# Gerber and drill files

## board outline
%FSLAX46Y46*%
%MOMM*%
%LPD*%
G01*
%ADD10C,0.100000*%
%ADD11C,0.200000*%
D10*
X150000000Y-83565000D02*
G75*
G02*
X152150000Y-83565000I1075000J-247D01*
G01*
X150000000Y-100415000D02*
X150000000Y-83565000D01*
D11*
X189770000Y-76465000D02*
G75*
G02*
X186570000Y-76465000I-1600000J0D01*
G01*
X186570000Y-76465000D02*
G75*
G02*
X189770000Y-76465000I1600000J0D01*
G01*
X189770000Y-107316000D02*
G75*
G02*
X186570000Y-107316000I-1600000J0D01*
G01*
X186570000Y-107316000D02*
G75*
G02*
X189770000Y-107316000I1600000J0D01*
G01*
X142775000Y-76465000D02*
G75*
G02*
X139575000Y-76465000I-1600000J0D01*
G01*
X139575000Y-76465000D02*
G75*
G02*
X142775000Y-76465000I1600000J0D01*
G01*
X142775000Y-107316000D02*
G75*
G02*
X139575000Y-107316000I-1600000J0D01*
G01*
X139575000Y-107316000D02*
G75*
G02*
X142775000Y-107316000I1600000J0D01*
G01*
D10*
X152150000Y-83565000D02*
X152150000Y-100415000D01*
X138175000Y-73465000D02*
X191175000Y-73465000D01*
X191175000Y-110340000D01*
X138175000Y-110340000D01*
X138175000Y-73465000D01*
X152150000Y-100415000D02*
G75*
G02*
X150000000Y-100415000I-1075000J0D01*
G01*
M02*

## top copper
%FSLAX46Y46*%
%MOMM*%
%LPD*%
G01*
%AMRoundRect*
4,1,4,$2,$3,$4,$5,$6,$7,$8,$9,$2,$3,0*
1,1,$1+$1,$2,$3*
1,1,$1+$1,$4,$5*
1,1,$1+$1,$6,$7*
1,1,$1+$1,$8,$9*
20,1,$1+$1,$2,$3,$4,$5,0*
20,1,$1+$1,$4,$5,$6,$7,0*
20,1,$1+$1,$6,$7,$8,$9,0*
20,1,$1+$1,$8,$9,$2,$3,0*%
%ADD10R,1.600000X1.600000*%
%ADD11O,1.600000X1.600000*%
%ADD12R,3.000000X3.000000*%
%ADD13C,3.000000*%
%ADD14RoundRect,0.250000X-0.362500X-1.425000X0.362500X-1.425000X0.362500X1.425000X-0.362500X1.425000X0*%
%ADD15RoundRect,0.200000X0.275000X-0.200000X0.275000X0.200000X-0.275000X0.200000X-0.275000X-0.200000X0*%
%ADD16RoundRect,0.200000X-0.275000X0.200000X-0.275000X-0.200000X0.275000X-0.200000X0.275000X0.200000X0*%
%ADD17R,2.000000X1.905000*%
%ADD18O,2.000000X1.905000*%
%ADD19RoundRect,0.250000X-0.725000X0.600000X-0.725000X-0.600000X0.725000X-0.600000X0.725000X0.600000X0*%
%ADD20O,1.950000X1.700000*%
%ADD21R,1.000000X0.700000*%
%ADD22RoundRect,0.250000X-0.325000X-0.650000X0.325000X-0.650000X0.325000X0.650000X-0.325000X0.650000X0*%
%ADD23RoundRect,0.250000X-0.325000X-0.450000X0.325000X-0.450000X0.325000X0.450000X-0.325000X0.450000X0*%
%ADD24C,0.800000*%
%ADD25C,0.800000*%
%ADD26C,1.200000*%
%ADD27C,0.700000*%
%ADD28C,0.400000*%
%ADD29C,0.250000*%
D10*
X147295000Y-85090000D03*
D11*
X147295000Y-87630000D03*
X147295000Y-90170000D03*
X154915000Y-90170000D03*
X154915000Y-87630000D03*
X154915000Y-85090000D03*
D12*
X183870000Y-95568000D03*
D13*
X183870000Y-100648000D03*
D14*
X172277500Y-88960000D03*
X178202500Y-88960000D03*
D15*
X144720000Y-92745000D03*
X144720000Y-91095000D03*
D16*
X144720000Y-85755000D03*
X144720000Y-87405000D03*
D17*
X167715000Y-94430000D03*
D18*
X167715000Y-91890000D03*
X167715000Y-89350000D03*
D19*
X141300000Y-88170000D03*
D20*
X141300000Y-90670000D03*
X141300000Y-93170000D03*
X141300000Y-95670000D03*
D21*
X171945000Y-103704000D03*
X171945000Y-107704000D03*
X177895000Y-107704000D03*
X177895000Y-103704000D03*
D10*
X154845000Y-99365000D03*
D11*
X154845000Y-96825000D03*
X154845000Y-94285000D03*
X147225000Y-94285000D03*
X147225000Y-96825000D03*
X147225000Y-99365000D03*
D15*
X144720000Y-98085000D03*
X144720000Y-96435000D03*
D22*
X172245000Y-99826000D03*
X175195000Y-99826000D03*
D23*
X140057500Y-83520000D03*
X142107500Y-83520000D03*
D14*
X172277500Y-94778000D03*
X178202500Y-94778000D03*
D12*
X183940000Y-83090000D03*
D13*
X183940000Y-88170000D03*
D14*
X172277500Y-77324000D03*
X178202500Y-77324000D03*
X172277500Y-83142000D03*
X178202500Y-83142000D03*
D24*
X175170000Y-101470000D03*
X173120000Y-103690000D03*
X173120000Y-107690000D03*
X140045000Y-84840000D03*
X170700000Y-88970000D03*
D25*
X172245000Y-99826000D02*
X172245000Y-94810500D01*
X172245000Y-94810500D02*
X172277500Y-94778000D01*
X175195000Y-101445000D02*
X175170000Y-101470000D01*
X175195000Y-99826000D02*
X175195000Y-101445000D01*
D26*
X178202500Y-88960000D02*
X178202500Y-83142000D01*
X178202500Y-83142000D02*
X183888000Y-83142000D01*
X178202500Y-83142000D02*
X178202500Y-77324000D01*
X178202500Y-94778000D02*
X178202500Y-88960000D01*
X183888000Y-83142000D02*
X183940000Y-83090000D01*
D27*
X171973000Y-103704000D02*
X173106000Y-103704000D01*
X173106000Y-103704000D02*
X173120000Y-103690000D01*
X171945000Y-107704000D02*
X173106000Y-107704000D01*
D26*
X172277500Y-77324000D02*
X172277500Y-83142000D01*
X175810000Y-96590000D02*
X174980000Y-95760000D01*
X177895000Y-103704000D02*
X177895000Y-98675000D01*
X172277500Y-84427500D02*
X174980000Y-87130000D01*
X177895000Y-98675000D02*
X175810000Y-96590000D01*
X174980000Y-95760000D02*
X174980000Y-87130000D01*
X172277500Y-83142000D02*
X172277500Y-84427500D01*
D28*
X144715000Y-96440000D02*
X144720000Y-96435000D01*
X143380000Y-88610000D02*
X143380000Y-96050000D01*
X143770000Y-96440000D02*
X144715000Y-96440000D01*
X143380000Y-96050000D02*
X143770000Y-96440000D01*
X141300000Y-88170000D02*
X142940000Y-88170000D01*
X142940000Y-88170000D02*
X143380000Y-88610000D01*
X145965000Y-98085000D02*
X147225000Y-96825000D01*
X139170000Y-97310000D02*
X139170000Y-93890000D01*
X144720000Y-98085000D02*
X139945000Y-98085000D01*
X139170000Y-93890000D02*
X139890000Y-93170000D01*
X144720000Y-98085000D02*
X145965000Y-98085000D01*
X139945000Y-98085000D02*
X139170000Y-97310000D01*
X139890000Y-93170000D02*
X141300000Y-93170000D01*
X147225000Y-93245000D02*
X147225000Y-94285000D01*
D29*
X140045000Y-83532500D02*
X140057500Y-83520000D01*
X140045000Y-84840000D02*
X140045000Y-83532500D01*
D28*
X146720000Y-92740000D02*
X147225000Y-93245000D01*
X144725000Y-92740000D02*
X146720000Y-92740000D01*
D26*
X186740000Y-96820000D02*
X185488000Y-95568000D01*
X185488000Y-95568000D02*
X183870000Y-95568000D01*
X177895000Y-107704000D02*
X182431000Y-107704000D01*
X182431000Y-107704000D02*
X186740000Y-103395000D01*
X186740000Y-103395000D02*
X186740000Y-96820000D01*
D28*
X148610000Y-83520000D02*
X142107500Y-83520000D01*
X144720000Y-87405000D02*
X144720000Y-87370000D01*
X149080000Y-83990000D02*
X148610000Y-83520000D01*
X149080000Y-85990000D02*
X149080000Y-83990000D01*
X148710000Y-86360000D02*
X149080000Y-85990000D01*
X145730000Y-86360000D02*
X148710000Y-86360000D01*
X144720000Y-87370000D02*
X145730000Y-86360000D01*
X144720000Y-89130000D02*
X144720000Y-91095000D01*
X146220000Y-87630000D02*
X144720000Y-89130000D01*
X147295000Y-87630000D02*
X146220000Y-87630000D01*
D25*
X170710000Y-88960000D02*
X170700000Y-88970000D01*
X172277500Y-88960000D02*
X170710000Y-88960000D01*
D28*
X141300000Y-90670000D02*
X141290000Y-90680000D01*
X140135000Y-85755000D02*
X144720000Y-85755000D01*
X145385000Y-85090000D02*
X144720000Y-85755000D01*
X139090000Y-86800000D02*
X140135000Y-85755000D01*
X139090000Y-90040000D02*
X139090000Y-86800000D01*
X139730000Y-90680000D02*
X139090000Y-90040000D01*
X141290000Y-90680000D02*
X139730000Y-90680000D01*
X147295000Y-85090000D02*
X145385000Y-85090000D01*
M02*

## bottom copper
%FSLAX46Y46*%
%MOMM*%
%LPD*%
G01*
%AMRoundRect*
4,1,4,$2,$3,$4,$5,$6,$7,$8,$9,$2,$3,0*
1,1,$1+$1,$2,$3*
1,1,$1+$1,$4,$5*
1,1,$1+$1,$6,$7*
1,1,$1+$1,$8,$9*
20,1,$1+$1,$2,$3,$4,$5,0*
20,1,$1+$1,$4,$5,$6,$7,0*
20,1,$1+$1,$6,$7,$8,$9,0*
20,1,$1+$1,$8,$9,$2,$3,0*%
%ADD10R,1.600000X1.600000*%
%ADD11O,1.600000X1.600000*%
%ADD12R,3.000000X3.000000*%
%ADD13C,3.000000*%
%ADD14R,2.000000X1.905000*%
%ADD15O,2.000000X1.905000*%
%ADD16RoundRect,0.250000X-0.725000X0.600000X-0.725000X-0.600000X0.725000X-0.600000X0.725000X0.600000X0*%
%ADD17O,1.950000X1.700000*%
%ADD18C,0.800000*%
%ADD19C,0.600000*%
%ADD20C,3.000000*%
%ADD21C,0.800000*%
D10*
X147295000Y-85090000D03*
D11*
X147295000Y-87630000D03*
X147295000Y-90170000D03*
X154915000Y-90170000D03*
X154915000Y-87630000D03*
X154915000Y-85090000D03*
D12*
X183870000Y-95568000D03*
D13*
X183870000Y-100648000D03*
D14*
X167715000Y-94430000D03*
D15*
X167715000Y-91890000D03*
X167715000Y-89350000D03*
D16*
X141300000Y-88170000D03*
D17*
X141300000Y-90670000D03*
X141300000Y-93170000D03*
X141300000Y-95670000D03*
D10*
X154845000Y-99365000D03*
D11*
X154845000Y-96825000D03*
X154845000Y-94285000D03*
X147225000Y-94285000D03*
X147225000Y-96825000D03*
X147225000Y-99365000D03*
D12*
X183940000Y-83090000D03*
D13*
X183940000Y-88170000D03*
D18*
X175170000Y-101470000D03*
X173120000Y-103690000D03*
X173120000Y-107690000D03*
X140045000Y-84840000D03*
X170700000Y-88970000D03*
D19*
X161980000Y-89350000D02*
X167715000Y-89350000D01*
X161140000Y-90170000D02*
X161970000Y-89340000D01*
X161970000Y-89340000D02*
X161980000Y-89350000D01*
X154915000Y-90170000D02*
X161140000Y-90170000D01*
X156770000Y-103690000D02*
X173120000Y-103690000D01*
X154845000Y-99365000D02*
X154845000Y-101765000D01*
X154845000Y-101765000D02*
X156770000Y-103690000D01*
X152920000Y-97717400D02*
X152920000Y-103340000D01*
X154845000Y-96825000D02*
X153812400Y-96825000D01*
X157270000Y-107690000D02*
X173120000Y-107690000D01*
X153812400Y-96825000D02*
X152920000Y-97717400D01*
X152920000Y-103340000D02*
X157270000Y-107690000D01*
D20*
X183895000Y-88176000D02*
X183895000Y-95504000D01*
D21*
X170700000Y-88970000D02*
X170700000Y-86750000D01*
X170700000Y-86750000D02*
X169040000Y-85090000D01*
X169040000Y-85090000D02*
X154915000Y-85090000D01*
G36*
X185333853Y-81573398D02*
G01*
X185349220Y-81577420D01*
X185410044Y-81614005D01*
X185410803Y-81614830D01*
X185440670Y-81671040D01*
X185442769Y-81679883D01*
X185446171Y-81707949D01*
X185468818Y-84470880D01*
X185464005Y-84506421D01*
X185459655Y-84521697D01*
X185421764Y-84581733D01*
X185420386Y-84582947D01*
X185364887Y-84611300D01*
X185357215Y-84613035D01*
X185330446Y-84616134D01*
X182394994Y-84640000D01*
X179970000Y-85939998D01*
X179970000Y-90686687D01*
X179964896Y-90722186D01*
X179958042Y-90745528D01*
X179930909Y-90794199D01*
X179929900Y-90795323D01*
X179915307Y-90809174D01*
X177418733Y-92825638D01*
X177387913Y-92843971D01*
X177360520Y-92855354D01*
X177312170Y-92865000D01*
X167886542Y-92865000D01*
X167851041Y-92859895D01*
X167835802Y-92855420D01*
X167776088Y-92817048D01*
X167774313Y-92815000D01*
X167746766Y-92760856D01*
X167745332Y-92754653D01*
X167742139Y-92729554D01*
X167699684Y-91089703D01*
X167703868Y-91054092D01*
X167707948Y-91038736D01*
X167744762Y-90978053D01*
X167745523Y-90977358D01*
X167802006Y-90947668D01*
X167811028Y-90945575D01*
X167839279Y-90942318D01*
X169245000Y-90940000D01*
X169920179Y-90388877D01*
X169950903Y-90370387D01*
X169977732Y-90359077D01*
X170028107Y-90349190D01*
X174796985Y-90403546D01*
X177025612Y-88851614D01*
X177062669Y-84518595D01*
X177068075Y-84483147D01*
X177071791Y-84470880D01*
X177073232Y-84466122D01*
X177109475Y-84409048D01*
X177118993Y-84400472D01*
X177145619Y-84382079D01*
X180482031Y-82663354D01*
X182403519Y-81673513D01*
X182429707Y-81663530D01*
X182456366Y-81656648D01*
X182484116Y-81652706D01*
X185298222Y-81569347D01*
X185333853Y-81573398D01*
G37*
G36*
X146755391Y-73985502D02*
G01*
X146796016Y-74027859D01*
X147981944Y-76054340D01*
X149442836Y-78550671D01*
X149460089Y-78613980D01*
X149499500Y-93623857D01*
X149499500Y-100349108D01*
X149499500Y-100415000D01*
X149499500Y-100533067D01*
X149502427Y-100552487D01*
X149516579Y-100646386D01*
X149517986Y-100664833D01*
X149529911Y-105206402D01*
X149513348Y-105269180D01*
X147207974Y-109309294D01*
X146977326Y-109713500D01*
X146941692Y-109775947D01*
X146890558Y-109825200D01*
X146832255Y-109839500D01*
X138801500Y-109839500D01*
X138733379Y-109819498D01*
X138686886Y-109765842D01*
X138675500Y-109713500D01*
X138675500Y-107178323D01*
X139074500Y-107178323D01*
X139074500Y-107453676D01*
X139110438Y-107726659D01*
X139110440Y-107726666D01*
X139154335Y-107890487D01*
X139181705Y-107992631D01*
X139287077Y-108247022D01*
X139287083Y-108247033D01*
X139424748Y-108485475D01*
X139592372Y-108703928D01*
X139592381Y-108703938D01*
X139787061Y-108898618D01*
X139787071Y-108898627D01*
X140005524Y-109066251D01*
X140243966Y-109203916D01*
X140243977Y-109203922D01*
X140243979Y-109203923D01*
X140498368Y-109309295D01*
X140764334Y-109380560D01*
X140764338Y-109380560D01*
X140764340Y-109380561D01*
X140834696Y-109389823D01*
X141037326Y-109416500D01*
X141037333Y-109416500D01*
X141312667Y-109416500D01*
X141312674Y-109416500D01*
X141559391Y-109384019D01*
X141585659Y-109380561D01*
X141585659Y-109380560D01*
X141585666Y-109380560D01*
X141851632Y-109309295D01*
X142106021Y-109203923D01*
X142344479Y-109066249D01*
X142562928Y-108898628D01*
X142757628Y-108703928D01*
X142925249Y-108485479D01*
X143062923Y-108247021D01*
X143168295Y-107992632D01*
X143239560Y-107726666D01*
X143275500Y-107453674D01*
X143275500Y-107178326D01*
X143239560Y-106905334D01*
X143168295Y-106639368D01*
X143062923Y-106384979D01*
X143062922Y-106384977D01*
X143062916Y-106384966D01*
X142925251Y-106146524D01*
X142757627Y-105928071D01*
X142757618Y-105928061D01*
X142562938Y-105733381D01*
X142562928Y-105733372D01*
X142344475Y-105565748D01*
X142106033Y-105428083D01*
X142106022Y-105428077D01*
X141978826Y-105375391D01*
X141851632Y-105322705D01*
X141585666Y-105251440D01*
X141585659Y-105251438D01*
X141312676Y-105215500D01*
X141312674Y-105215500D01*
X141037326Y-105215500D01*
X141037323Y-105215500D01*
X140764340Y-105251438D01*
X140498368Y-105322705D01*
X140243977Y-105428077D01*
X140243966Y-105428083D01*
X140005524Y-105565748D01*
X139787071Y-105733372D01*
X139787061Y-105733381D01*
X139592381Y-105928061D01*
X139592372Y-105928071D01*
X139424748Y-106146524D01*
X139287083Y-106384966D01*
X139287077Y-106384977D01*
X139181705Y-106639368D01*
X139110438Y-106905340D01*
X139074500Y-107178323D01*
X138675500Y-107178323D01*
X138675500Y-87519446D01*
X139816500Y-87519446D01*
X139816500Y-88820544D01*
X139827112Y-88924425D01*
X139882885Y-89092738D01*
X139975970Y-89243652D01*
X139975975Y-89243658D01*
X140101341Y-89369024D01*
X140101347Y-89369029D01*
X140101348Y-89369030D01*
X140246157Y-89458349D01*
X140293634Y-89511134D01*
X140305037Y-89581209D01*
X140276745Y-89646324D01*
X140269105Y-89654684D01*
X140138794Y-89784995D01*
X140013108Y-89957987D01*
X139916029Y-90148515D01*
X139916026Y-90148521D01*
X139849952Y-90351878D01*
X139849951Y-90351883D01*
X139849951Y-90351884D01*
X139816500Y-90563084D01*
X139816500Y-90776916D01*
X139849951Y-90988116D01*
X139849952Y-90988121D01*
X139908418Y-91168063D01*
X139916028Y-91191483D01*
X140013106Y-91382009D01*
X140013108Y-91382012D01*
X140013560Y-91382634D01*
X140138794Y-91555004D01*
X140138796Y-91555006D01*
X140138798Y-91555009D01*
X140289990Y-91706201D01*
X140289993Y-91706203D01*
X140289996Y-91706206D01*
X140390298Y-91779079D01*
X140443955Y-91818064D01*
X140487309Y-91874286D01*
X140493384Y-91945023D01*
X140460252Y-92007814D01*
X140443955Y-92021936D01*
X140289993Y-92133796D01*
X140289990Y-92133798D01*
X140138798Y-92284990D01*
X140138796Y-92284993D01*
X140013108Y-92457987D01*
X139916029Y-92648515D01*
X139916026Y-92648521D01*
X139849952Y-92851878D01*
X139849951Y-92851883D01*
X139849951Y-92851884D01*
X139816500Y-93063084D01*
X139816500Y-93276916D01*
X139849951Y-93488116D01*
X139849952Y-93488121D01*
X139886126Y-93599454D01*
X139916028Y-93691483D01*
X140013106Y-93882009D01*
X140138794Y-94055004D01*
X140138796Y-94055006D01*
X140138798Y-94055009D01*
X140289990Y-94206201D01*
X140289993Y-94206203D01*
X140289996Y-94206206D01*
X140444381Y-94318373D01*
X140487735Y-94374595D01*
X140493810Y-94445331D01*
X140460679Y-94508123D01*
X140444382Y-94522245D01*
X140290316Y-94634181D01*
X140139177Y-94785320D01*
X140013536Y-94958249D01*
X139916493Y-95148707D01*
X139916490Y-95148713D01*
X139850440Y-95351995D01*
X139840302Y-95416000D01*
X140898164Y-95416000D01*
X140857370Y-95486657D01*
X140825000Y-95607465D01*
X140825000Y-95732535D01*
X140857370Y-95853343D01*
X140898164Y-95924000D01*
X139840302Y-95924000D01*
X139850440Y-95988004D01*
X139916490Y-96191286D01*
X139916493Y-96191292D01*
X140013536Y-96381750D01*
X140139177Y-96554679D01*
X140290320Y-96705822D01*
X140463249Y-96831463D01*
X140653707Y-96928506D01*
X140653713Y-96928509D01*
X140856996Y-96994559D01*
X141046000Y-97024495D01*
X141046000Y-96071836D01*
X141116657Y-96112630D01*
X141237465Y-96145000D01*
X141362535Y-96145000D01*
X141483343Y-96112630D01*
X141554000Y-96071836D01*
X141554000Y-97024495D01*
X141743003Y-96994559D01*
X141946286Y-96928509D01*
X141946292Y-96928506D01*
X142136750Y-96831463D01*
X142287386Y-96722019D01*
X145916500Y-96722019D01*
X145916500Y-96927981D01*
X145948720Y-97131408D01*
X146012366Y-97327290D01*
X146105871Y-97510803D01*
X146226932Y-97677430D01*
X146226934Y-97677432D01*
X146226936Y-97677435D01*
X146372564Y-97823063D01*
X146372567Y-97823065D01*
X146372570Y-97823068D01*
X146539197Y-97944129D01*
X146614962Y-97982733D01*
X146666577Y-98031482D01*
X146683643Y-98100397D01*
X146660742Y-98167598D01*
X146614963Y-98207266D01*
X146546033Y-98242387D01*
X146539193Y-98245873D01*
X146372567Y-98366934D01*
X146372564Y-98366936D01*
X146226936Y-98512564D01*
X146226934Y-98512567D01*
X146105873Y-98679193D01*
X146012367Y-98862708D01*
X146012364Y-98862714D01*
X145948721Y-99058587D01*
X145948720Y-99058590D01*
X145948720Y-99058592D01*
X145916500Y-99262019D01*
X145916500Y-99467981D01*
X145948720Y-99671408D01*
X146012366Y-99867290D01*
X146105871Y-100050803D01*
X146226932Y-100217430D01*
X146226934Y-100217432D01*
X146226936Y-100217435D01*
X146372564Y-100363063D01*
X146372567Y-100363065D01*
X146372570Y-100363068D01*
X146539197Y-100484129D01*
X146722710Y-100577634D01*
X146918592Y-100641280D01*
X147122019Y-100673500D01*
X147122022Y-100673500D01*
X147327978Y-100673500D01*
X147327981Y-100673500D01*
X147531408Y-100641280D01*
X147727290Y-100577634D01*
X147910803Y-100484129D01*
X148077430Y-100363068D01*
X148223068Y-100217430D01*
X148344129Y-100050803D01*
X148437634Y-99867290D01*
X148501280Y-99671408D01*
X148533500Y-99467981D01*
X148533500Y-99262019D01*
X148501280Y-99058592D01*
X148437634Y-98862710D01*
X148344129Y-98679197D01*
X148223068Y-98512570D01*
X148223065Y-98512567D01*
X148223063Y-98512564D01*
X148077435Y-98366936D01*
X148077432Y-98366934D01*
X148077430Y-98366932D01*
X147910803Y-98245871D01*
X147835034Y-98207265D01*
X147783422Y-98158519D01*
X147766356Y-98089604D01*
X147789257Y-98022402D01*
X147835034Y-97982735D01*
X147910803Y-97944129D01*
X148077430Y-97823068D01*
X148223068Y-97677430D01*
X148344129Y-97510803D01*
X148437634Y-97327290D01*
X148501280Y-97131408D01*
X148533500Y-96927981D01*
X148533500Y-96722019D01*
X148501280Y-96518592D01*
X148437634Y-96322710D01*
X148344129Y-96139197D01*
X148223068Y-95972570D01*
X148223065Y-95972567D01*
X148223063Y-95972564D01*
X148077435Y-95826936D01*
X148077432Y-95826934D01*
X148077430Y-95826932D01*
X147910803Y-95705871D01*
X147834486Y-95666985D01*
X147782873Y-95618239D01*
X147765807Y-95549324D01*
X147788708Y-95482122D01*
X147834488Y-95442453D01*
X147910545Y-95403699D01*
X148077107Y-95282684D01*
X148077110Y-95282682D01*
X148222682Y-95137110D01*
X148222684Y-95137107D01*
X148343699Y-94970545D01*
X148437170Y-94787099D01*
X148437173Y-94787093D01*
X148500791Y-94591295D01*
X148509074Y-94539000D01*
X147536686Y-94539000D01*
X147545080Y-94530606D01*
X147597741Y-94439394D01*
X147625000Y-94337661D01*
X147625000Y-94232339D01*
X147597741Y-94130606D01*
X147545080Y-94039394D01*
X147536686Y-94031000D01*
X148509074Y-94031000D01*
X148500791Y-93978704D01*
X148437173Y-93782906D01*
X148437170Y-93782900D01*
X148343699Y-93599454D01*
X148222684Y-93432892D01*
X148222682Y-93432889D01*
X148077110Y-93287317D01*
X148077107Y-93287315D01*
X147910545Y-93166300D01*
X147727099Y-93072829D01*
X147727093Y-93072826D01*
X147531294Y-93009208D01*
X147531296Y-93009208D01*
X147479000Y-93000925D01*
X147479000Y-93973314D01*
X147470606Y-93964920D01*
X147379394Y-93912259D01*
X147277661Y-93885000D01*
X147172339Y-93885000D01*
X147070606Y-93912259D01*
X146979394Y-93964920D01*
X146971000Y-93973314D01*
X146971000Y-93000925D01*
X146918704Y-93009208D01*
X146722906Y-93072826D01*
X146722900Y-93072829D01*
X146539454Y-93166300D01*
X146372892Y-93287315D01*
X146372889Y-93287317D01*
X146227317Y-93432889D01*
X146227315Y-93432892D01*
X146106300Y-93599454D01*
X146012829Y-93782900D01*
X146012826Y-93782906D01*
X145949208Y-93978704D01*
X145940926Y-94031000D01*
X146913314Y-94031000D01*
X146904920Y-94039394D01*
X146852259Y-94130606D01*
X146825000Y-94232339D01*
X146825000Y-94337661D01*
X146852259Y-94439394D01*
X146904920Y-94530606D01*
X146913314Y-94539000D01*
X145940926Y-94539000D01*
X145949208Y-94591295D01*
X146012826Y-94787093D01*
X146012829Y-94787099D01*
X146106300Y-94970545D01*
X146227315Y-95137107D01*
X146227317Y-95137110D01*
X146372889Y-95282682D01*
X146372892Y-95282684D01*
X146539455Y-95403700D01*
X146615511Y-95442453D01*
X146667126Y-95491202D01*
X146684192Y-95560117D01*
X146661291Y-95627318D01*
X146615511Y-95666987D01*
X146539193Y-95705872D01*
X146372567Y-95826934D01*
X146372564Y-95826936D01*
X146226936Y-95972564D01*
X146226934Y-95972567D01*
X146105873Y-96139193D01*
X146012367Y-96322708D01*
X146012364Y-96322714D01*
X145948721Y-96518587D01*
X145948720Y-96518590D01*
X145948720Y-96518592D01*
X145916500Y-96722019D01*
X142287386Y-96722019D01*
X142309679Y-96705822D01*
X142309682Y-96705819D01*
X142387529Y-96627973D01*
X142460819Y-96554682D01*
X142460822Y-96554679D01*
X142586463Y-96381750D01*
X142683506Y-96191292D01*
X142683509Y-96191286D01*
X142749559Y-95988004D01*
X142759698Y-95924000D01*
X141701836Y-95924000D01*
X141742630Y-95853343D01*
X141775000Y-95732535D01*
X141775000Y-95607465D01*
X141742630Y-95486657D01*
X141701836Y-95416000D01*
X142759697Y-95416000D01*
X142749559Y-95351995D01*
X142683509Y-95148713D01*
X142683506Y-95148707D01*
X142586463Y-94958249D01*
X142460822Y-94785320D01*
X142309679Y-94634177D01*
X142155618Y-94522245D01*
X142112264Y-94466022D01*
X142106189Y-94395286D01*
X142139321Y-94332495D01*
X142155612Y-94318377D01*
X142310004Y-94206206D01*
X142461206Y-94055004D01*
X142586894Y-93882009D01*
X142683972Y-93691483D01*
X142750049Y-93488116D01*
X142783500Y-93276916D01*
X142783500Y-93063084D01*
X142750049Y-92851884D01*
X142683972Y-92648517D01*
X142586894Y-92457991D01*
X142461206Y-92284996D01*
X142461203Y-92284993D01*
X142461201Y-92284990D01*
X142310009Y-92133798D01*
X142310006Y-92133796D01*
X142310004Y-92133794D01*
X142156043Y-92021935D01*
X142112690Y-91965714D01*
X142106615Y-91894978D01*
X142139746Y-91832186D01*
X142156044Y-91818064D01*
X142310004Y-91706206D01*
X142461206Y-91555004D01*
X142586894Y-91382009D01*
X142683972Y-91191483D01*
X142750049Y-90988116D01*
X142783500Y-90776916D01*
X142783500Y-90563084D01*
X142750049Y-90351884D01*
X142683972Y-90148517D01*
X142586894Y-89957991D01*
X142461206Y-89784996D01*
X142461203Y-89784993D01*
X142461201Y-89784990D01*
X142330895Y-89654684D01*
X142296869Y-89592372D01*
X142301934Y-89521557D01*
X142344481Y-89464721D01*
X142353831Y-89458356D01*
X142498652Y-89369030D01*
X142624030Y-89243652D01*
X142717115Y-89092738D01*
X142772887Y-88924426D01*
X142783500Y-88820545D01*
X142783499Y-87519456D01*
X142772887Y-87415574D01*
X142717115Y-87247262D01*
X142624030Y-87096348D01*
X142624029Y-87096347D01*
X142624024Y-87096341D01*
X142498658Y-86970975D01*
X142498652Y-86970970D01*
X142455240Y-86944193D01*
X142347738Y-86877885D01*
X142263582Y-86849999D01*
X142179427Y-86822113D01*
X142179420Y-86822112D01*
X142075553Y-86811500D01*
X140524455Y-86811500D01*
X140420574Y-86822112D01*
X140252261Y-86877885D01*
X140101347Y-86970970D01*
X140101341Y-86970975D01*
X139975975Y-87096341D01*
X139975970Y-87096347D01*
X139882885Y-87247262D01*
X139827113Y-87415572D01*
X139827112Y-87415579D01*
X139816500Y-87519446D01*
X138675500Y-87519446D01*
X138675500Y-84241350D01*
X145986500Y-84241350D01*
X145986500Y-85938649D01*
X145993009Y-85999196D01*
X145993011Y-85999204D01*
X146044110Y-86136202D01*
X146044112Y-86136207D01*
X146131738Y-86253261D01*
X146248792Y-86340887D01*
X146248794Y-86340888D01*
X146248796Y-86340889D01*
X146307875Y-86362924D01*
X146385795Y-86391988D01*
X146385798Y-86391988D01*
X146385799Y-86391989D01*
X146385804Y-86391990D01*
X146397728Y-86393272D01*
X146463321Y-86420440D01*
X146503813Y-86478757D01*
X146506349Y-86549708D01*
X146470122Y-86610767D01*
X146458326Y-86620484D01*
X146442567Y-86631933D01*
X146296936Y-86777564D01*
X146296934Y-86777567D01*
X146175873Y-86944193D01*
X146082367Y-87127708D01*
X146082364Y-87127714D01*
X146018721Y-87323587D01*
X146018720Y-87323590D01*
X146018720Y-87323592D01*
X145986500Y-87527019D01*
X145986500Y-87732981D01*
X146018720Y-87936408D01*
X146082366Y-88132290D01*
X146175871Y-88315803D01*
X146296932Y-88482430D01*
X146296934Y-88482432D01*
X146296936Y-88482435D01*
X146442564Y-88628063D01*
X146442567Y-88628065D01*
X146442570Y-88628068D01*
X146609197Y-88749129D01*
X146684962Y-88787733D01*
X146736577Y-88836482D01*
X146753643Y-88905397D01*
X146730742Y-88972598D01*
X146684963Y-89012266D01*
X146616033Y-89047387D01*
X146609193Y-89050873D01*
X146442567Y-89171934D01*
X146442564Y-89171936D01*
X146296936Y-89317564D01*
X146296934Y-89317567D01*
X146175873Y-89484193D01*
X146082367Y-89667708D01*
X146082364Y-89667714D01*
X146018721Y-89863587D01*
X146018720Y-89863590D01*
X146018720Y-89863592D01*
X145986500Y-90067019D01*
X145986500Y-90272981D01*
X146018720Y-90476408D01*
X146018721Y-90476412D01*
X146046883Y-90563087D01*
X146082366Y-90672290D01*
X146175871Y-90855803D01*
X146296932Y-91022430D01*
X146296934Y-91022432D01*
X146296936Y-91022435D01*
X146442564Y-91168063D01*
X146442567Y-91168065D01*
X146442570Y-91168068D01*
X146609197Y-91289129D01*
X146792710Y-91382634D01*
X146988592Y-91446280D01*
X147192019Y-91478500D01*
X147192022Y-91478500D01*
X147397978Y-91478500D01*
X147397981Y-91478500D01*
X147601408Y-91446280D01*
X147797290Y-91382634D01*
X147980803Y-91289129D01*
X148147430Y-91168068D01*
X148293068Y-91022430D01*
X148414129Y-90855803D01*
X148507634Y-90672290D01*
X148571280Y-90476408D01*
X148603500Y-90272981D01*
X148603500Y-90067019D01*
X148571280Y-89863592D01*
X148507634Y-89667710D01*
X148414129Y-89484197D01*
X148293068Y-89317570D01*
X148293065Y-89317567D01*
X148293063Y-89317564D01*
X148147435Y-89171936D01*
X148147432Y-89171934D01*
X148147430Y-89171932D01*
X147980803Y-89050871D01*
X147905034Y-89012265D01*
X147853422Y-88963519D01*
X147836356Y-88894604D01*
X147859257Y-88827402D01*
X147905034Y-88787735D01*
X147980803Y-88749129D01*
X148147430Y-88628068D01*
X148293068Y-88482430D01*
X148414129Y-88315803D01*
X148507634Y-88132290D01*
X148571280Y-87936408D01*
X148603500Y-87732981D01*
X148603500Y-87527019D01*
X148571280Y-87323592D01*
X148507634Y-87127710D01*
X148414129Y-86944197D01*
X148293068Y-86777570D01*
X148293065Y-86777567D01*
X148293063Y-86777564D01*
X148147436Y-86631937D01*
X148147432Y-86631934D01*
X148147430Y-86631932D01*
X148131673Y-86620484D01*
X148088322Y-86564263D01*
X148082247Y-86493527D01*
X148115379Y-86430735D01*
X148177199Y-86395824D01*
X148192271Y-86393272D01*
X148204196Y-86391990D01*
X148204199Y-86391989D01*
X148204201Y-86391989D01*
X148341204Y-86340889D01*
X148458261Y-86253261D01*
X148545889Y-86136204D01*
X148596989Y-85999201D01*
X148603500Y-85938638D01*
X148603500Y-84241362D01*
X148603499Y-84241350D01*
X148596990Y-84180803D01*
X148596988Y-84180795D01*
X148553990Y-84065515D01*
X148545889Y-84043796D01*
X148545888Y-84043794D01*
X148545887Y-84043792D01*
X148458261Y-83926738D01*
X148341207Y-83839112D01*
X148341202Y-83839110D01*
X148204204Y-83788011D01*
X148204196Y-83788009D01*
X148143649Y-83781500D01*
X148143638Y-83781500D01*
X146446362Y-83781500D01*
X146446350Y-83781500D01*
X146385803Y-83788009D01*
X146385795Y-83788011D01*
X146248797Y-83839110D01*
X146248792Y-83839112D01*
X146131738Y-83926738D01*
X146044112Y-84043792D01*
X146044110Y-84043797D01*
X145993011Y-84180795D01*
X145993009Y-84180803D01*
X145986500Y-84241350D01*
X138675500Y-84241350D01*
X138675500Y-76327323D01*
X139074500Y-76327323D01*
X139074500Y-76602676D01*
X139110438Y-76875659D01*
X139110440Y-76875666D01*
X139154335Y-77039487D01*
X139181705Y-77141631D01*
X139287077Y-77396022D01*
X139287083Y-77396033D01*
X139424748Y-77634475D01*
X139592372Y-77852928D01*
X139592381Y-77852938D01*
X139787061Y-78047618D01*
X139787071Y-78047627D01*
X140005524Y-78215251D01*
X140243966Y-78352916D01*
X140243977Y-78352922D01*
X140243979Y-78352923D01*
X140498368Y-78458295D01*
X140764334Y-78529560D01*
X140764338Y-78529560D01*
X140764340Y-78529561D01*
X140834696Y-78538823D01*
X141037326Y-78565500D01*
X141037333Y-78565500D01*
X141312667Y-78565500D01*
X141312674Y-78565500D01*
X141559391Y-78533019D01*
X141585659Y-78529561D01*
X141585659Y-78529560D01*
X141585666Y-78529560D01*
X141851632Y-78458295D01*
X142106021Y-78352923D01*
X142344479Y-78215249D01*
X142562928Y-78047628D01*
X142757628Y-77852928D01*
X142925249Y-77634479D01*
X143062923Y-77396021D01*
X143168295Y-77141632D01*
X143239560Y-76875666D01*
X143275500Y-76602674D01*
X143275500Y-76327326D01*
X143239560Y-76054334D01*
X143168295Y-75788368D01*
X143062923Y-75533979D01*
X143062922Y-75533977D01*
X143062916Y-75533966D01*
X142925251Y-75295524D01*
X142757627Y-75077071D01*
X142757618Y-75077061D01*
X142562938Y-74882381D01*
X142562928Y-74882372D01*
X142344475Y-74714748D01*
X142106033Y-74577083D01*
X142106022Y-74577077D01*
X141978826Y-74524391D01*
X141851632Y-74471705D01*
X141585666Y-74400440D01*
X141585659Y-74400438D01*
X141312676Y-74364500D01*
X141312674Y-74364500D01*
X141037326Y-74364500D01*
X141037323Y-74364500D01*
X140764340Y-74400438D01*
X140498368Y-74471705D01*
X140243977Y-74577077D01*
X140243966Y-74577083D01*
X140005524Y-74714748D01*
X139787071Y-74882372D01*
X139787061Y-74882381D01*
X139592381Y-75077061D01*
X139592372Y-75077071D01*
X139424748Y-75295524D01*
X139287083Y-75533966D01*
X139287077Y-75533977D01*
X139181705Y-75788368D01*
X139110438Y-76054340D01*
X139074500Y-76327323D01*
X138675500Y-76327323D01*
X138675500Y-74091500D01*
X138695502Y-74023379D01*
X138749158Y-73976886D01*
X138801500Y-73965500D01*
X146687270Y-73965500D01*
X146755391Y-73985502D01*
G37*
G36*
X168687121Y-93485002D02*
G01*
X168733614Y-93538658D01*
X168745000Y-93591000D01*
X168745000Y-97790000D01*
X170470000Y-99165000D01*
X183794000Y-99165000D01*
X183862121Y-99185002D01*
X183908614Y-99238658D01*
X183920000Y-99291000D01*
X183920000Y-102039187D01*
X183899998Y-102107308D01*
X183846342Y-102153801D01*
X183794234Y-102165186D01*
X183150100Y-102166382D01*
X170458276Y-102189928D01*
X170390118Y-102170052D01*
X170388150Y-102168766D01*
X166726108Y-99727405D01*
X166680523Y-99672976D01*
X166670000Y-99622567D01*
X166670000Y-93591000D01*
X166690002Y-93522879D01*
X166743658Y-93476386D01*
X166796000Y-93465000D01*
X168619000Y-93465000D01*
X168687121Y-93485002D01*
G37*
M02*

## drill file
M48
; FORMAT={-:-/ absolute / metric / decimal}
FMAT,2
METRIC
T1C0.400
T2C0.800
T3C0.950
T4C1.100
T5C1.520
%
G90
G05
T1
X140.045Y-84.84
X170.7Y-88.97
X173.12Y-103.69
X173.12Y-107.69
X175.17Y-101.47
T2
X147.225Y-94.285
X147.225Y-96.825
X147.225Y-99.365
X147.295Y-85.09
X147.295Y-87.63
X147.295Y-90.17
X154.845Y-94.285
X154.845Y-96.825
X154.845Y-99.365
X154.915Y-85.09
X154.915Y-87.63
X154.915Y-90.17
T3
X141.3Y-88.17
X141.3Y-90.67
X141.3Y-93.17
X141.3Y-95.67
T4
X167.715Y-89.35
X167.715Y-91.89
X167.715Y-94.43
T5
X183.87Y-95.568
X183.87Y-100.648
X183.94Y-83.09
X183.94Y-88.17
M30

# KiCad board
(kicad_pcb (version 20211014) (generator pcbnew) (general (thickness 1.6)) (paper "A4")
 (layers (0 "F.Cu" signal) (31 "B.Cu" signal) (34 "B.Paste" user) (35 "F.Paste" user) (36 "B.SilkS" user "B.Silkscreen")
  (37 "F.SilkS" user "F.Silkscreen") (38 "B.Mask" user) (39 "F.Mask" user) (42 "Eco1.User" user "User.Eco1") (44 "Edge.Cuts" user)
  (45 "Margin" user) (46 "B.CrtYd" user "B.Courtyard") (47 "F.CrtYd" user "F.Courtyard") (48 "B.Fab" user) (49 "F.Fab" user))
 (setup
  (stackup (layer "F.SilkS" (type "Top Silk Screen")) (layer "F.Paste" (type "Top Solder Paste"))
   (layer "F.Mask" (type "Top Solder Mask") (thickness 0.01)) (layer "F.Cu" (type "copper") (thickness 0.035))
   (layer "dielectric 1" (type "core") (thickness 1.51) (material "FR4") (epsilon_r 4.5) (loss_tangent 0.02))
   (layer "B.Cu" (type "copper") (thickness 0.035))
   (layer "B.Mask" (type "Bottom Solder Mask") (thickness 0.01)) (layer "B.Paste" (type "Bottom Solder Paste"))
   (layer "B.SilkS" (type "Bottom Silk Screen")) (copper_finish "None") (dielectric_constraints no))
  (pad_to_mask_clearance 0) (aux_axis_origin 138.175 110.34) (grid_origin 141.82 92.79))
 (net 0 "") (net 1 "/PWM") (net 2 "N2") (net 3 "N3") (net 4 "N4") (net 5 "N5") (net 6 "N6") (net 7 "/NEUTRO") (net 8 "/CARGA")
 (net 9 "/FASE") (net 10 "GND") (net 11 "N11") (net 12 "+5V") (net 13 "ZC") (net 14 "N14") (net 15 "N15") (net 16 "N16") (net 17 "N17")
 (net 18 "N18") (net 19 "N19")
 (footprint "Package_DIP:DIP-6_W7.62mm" (layer "F.Cu") (at 147.295 85.09)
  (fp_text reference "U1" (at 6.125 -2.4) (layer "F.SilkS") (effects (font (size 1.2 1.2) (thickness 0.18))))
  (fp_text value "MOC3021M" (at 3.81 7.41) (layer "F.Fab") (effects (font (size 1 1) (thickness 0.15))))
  (pad "1" thru_hole rect (at 0 0) (size 1.6 1.6) (drill 0.8) (layers *.Cu *.Mask) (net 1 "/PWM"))
  (pad "2" thru_hole oval (at 0 2.54) (size 1.6 1.6) (drill 0.8) (layers *.Cu *.Mask) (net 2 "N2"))
  (pad "3" thru_hole oval (at 0 5.08) (size 1.6 1.6) (drill 0.8) (layers *.Cu *.Mask) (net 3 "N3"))
  (pad "4" thru_hole oval (at 7.62 5.08) (size 1.6 1.6) (drill 0.8) (layers *.Cu *.Mask) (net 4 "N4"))
  (pad "5" thru_hole oval (at 7.62 2.54) (size 1.6 1.6) (drill 0.8) (layers *.Cu *.Mask) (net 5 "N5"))
  (pad "6" thru_hole oval (at 7.62 0) (size 1.6 1.6) (drill 0.8) (layers *.Cu *.Mask) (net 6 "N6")))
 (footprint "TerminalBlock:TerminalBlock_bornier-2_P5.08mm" (layer "F.Cu") (at 183.87 95.568 -90)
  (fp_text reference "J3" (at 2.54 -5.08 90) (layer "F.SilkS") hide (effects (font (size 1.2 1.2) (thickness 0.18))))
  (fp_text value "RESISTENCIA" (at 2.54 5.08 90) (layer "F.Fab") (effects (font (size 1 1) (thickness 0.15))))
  (pad "1" thru_hole rect (at 0 0 270) (size 3 3) (drill 1.52) (layers *.Cu *.Mask) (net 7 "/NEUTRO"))
  (pad "2" thru_hole circle (at 5.08 0 270) (size 3 3) (drill 1.52) (layers *.Cu *.Mask) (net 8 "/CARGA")))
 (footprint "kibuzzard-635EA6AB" (layer "F.Cu") (at 141.02 81.09)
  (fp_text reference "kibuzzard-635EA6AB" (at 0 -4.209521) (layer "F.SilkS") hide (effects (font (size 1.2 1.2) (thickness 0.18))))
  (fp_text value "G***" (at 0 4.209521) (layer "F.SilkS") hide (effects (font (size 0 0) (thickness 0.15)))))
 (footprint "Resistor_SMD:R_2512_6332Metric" (layer "F.Cu") (at 175.24 88.96)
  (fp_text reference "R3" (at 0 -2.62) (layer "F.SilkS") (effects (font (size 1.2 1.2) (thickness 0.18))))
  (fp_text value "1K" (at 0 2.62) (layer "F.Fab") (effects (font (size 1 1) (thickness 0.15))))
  (pad "1" smd roundrect (at -2.9625 0) (size 1.225 3.35) (layers "F.Cu" "F.Paste" "F.Mask") (roundrect_rratio 0.204082) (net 6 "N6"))
  (pad "2" smd roundrect (at 2.9625 0) (size 1.225 3.35) (layers "F.Cu" "F.Paste" "F.Mask") (roundrect_rratio 0.204082) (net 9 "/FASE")))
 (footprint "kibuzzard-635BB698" (layer "F.Cu") (at 189.41619 85.8 90)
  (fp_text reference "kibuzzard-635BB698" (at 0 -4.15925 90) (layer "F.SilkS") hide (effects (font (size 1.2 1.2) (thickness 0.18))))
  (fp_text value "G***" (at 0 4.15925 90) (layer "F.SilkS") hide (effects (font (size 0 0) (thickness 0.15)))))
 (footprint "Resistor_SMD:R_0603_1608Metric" (layer "F.Cu") (at 144.72 91.92 90)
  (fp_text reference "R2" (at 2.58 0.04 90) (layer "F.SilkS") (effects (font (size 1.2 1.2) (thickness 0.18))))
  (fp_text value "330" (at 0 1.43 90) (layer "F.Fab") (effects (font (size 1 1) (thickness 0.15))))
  (pad "1" smd roundrect (at -0.825 0 90) (size 0.8 0.95) (layers "F.Cu" "F.Paste" "F.Mask") (roundrect_rratio 0.25) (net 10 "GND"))
  (pad "2" smd roundrect (at 0.825 0 90) (size 0.8 0.95) (layers "F.Cu" "F.Paste" "F.Mask") (roundrect_rratio 0.25) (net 2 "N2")))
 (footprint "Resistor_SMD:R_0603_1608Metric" (layer "F.Cu") (at 144.72 86.58 -90)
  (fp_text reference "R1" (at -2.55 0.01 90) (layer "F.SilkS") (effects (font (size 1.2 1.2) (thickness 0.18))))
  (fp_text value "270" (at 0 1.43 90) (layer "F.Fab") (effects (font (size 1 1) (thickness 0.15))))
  (pad "1" smd roundrect (at -0.825 0 270) (size 0.8 0.95) (layers "F.Cu" "F.Paste" "F.Mask") (roundrect_rratio 0.25) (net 1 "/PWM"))
  (pad "2" smd roundrect (at 0.825 0 270) (size 0.8 0.95) (layers "F.Cu" "F.Paste" "F.Mask") (roundrect_rratio 0.25) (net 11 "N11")))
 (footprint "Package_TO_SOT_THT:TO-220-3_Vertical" (layer "F.Cu") (at 167.715 94.43 90)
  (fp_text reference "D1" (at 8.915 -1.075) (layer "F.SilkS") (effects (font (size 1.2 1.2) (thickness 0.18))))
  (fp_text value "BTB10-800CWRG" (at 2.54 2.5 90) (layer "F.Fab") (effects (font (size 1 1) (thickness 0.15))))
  (pad "1" thru_hole rect (at 0 0 90) (size 1.905 2) (drill 1.1) (layers *.Cu *.Mask) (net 8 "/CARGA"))
  (pad "2" thru_hole oval (at 2.54 0 90) (size 1.905 2) (drill 1.1) (layers *.Cu *.Mask) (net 9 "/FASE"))
  (pad "3" thru_hole oval (at 5.08 0 90) (size 1.905 2) (drill 1.1) (layers *.Cu *.Mask) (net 4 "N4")))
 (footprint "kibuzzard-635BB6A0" (layer "F.Cu") (at 189.42 98.01 90)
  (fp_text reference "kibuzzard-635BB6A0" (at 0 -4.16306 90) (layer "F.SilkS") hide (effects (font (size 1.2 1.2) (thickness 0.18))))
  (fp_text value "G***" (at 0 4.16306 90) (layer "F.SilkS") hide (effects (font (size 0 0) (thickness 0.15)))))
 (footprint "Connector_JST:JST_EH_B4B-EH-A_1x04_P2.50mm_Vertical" (layer "F.Cu") (at 141.3 88.17 -90)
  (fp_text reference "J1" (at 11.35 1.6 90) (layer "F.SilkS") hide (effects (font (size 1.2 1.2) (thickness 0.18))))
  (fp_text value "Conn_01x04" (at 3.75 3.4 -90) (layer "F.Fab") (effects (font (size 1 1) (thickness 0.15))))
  (pad "1" thru_hole roundrect (at 0 0 270) (size 1.7 1.95) (drill 0.95) (layers *.Cu *.Mask) (roundrect_rratio 0.147059) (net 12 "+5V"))
  (pad "2" thru_hole oval (at 2.5 0 270) (size 1.7 1.95) (drill 0.95) (layers *.Cu *.Mask) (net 1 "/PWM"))
  (pad "3" thru_hole oval (at 5 0 270) (size 1.7 1.95) (drill 0.95) (layers *.Cu *.Mask) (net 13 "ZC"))
  (pad "4" thru_hole oval (at 7.5 0 270) (size 1.7 1.95) (drill 0.95) (layers *.Cu *.Mask) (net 10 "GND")))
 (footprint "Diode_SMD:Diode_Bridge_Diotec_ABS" (layer "F.Cu") (at 174.92 105.704)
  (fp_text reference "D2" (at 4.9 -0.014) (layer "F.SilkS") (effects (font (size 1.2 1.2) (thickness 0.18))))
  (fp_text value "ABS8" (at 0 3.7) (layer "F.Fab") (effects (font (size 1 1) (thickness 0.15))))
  (pad "1" smd rect (at -2.975 -2) (size 1 0.7) (layers "F.Cu" "F.Paste" "F.Mask") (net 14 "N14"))
  (pad "2" smd rect (at -2.975 2) (size 1 0.7) (layers "F.Cu" "F.Paste" "F.Mask") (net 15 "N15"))
  (pad "3" smd rect (at 2.975 2) (size 1 0.7) (layers "F.Cu" "F.Paste" "F.Mask") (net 7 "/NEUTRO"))
  (pad "4" smd rect (at 2.975 -2) (size 1 0.7) (layers "F.Cu" "F.Paste" "F.Mask") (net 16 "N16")))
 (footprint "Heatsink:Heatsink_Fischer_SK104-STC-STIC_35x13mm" (layer "F.Cu") (at 163.48 91.96 90)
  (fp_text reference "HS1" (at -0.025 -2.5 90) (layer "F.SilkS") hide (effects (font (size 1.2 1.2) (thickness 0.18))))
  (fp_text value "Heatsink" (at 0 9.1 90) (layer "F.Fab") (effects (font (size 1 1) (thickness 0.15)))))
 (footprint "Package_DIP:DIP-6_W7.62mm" (layer "F.Cu") (at 154.845 99.365 180)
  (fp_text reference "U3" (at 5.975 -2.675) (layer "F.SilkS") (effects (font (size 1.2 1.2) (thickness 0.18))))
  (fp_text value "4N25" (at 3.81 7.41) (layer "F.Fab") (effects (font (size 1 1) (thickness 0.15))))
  (pad "1" thru_hole rect (at 0 0 180) (size 1.6 1.6) (drill 0.8) (layers *.Cu *.Mask) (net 14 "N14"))
  (pad "2" thru_hole oval (at 0 2.54 180) (size 1.6 1.6) (drill 0.8) (layers *.Cu *.Mask) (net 15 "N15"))
  (pad "3" thru_hole oval (at 0 5.08 180) (size 1.6 1.6) (drill 0.8) (layers *.Cu *.Mask) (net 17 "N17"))
  (pad "4" thru_hole oval (at 7.62 5.08 180) (size 1.6 1.6) (drill 0.8) (layers *.Cu *.Mask) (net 10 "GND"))
  (pad "5" thru_hole oval (at 7.62 2.54 180) (size 1.6 1.6) (drill 0.8) (layers *.Cu *.Mask) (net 13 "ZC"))
  (pad "6" thru_hole oval (at 7.62 0 180) (size 1.6 1.6) (drill 0.8) (layers *.Cu *.Mask) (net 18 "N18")))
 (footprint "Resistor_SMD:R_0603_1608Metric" (layer "F.Cu") (at 144.72 97.26 90)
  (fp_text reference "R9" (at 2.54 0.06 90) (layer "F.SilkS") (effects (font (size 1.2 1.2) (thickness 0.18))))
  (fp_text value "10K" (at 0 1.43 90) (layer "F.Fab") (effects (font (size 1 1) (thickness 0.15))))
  (pad "1" smd roundrect (at -0.825 0 90) (size 0.8 0.95) (layers "F.Cu" "F.Paste" "F.Mask") (roundrect_rratio 0.25) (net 13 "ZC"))
  (pad "2" smd roundrect (at 0.825 0 90) (size 0.8 0.95) (layers "F.Cu" "F.Paste" "F.Mask") (roundrect_rratio 0.25) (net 12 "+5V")))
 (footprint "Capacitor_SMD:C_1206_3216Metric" (layer "F.Cu") (at 173.72 99.826)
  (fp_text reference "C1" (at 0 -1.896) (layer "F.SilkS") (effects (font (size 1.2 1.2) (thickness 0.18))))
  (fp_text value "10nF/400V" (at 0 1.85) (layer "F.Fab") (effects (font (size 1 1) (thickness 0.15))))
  (pad "1" smd roundrect (at -1.475 0) (size 1.15 1.8) (layers "F.Cu" "F.Paste" "F.Mask") (roundrect_rratio 0.217391) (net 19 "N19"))
  (pad "2" smd roundrect (at 1.475 0) (size 1.15 1.8) (layers "F.Cu" "F.Paste" "F.Mask") (roundrect_rratio 0.217391) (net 8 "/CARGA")))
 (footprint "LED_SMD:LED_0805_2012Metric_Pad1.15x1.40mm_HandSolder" (layer "F.Cu") (at 141.0825 83.52)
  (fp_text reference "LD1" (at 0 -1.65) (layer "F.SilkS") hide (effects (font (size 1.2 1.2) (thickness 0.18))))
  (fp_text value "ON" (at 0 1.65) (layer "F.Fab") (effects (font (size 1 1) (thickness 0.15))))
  (pad "1" smd roundrect (at -1.025 0) (size 1.15 1.4) (layers "F.Cu" "F.Paste" "F.Mask") (roundrect_rratio 0.217391) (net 10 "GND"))
  (pad "2" smd roundrect (at 1.025 0) (size 1.15 1.4) (layers "F.Cu" "F.Paste" "F.Mask") (roundrect_rratio 0.217391) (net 11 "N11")))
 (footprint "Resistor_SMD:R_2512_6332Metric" (layer "F.Cu") (at 175.24 94.778)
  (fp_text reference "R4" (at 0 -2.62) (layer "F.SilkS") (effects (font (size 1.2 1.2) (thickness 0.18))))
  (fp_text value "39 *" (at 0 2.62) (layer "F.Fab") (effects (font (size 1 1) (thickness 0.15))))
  (pad "1" smd roundrect (at -2.9625 0) (size 1.225 3.35) (layers "F.Cu" "F.Paste" "F.Mask") (roundrect_rratio 0.204082) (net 19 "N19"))
  (pad "2" smd roundrect (at 2.9625 0) (size 1.225 3.35) (layers "F.Cu" "F.Paste" "F.Mask") (roundrect_rratio 0.204082) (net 9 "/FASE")))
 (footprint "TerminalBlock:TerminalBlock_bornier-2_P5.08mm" (layer "F.Cu") (at 183.94 83.09 -90)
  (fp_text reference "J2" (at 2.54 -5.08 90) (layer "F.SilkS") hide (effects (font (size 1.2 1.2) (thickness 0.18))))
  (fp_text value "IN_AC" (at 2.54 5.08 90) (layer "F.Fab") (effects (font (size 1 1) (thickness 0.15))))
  (pad "1" thru_hole rect (at 0 0 270) (size 3 3) (drill 1.52) (layers *.Cu *.Mask) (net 9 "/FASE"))
  (pad "2" thru_hole circle (at 5.08 0 270) (size 3 3) (drill 1.52) (layers *.Cu *.Mask) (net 7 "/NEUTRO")))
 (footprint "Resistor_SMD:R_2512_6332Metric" (layer "F.Cu") (at 175.24 77.324)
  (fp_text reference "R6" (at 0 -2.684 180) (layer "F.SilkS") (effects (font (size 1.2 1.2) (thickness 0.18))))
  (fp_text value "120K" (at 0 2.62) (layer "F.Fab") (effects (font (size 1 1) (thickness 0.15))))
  (pad "1" smd roundrect (at -2.9625 0) (size 1.225 3.35) (layers "F.Cu" "F.Paste" "F.Mask") (roundrect_rratio 0.204082) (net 16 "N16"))
  (pad "2" smd roundrect (at 2.9625 0) (size 1.225 3.35) (layers "F.Cu" "F.Paste" "F.Mask") (roundrect_rratio 0.204082) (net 9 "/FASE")))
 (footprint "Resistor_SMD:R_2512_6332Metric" (layer "F.Cu") (at 175.24 83.142)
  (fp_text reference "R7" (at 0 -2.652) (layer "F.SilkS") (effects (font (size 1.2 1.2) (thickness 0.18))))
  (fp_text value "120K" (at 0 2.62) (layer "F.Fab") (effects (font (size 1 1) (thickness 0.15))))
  (pad "1" smd roundrect (at -2.9625 0) (size 1.225 3.35) (layers "F.Cu" "F.Paste" "F.Mask") (roundrect_rratio 0.204082) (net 16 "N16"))
  (pad "2" smd roundrect (at 2.9625 0) (size 1.225 3.35) (layers "F.Cu" "F.Paste" "F.Mask") (roundrect_rratio 0.204082) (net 9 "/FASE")))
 (gr_arc (start 150 83.565) (mid 151.075 82.490247) (end 152.15 83.565) (layer "Edge.Cuts") (width 0.1))
 (gr_line (start 150 100.415) (end 150 83.565) (layer "Edge.Cuts") (width 0.1))
 (gr_circle (center 188.17 76.465) (end 189.77 76.465) (layer "Edge.Cuts") (width 0.2) (fill none))
 (gr_circle (center 188.17 107.316) (end 189.77 107.316) (layer "Edge.Cuts") (width 0.2) (fill none))
 (gr_circle (center 141.175 76.465) (end 142.775 76.465) (layer "Edge.Cuts") (width 0.2) (fill none))
 (gr_circle (center 141.175 107.316) (end 142.775 107.316) (layer "Edge.Cuts") (width 0.2) (fill none))
 (gr_line (start 152.15 83.565) (end 152.15 100.415) (layer "Edge.Cuts") (width 0.1))
 (gr_rect (start 138.175 73.465) (end 191.175 110.34) (layer "Edge.Cuts") (width 0.1) (fill none))
 (gr_arc (start 152.15 100.415) (mid 151.075 101.49) (end 150 100.415) (layer "Edge.Cuts") (width 0.1))
 (segment (start 172.245 99.826) (end 172.245 94.8105) (width 0.8) (layer "F.Cu") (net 19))
 (segment (start 172.245 94.8105) (end 172.2775 94.778) (width 0.8) (layer "F.Cu") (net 19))
 (segment (start 175.195 101.445) (end 175.17 101.47) (width 0.8) (layer "F.Cu") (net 8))
 (segment (start 175.195 99.826) (end 175.195 101.445) (width 0.8) (layer "F.Cu") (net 8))
 (via (at 175.17 101.47) (size 0.8) (drill 0.4) (layers "F.Cu" "B.Cu") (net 8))
 (segment (start 178.2025 88.96) (end 178.2025 83.142) (width 1.2) (layer "F.Cu") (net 9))
 (segment (start 178.2025 83.142) (end 183.888 83.142) (width 1.2) (layer "F.Cu") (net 9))
 (segment (start 178.2025 83.142) (end 178.2025 77.324) (width 1.2) (layer "F.Cu") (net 9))
 (segment (start 178.2025 94.778) (end 178.2025 88.96) (width 1.2) (layer "F.Cu") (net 9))
 (segment (start 183.888 83.142) (end 183.94 83.09) (width 1.2) (layer "F.Cu") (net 9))
 (segment (start 161.98 89.35) (end 167.715 89.35) (width 0.6) (layer "B.Cu") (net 4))
 (segment (start 161.14 90.17) (end 161.97 89.34) (width 0.6) (layer "B.Cu") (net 4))
 (segment (start 161.97 89.34) (end 161.98 89.35) (width 0.6) (layer "B.Cu") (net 4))
 (segment (start 154.915 90.17) (end 161.14 90.17) (width 0.6) (layer "B.Cu") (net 4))
 (segment (start 171.973 103.704) (end 173.106 103.704) (width 0.7) (layer "F.Cu") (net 14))
 (segment (start 173.106 103.704) (end 173.12 103.69) (width 0.7) (layer "F.Cu") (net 14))
 (via (at 173.12 103.69) (size 0.8) (drill 0.4) (layers "F.Cu" "B.Cu") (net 14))
 (segment (start 156.77 103.69) (end 173.12 103.69) (width 0.6) (layer "B.Cu") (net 14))
 (segment (start 154.845 99.365) (end 154.845 101.765) (width 0.6) (layer "B.Cu") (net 14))
 (segment (start 154.845 101.765) (end 156.77 103.69) (width 0.6) (layer "B.Cu") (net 14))
 (segment (start 171.945 107.704) (end 173.106 107.704) (width 0.7) (layer "F.Cu") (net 15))
 (via (at 173.12 107.69) (size 0.8) (drill 0.4) (layers "F.Cu" "B.Cu") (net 15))
 (segment (start 152.92 97.7174) (end 152.92 103.34) (width 0.6) (layer "B.Cu") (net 15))
 (segment (start 154.845 96.825) (end 153.8124 96.825) (width 0.6) (layer "B.Cu") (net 15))
 (segment (start 157.27 107.69) (end 173.12 107.69) (width 0.6) (layer "B.Cu") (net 15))
 (segment (start 153.8124 96.825) (end 152.92 97.7174) (width 0.6) (layer "B.Cu") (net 15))
 (segment (start 152.92 103.34) (end 157.27 107.69) (width 0.6) (layer "B.Cu") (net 15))
 (segment (start 172.2775 77.324) (end 172.2775 83.142) (width 1.2) (layer "F.Cu") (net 16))
 (segment (start 175.81 96.59) (end 174.98 95.76) (width 1.2) (layer "F.Cu") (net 16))
 (segment (start 177.895 103.704) (end 177.895 98.675) (width 1.2) (layer "F.Cu") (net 16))
 (segment (start 172.2775 84.4275) (end 174.98 87.13) (width 1.2) (layer "F.Cu") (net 16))
 (segment (start 177.895 98.675) (end 175.81 96.59) (width 1.2) (layer "F.Cu") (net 16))
 (segment (start 174.98 95.76) (end 174.98 87.13) (width 1.2) (layer "F.Cu") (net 16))
 (segment (start 172.2775 83.142) (end 172.2775 84.4275) (width 1.2) (layer "F.Cu") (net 16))
 (segment (start 144.715 96.44) (end 144.72 96.435) (width 0.4) (layer "F.Cu") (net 12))
 (segment (start 143.38 88.61) (end 143.38 96.05) (width 0.4) (layer "F.Cu") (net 12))
 (segment (start 143.77 96.44) (end 144.715 96.44) (width 0.4) (layer "F.Cu") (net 12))
 (segment (start 143.38 96.05) (end 143.77 96.44) (width 0.4) (layer "F.Cu") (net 12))
 (segment (start 141.3 88.17) (end 142.94 88.17) (width 0.4) (layer "F.Cu") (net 12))
 (segment (start 142.94 88.17) (end 143.38 88.61) (width 0.4) (layer "F.Cu") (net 12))
 (segment (start 145.965 98.085) (end 147.225 96.825) (width 0.4) (layer "F.Cu") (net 13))
 (segment (start 139.17 97.31) (end 139.17 93.89) (width 0.4) (layer "F.Cu") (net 13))
 (segment (start 144.72 98.085) (end 139.945 98.085) (width 0.4) (layer "F.Cu") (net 13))
 (segment (start 139.17 93.89) (end 139.89 93.17) (width 0.4) (layer "F.Cu") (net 13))
 (segment (start 144.72 98.085) (end 145.965 98.085) (width 0.4) (layer "F.Cu") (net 13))
 (segment (start 139.945 98.085) (end 139.17 97.31) (width 0.4) (layer "F.Cu") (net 13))
 (segment (start 139.89 93.17) (end 141.3 93.17) (width 0.4) (layer "F.Cu") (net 13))
 (segment (start 147.225 93.245) (end 147.225 94.285) (width 0.4) (layer "F.Cu") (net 10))
 (segment (start 140.045 83.5325) (end 140.0575 83.52) (width 0.25) (layer "F.Cu") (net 10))
 (segment (start 140.045 84.84) (end 140.045 83.5325) (width 0.25) (layer "F.Cu") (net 10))
 (segment (start 146.72 92.74) (end 147.225 93.245) (width 0.4) (layer "F.Cu") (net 10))
 (segment (start 144.725 92.74) (end 146.72 92.74) (width 0.4) (layer "F.Cu") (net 10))
 (via (at 140.045 84.84) (size 0.8) (drill 0.4) (layers "F.Cu" "B.Cu") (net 10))
 (segment (start 186.74 96.82) (end 185.488 95.568) (width 1.2) (layer "F.Cu") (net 7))
 (segment (start 185.488 95.568) (end 183.87 95.568) (width 1.2) (layer "F.Cu") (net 7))
 (segment (start 177.895 107.704) (end 182.431 107.704) (width 1.2) (layer "F.Cu") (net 7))
 (segment (start 182.431 107.704) (end 186.74 103.395) (width 1.2) (layer "F.Cu") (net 7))
 (segment (start 186.74 103.395) (end 186.74 96.82) (width 1.2) (layer "F.Cu") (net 7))
 (segment (start 183.895 88.176) (end 183.895 95.504) (width 3) (layer "B.Cu") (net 7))
 (segment (start 148.61 83.52) (end 142.1075 83.52) (width 0.4) (layer "F.Cu") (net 11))
 (segment (start 144.72 87.405) (end 144.72 87.37) (width 0.4) (layer "F.Cu") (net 11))
 (segment (start 149.08 83.99) (end 148.61 83.52) (width 0.4) (layer "F.Cu") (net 11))
 (segment (start 149.08 85.99) (end 149.08 83.99) (width 0.4) (layer "F.Cu") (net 11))
 (segment (start 148.71 86.36) (end 149.08 85.99) (width 0.4) (layer "F.Cu") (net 11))
 (segment (start 145.73 86.36) (end 148.71 86.36) (width 0.4) (layer "F.Cu") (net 11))
 (segment (start 144.72 87.37) (end 145.73 86.36) (width 0.4) (layer "F.Cu") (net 11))
 (segment (start 144.72 89.13) (end 144.72 91.095) (width 0.4) (layer "F.Cu") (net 2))
 (segment (start 146.22 87.63) (end 144.72 89.13) (width 0.4) (layer "F.Cu") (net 2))
 (segment (start 147.295 87.63) (end 146.22 87.63) (width 0.4) (layer "F.Cu") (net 2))
 (segment (start 170.71 88.96) (end 170.7 88.97) (width 0.8) (layer "F.Cu") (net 6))
 (segment (start 172.2775 88.96) (end 170.71 88.96) (width 0.8) (layer "F.Cu") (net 6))
 (via (at 170.7 88.97) (size 0.8) (drill 0.4) (layers "F.Cu" "B.Cu") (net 6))
 (segment (start 170.7 88.97) (end 170.7 86.75) (width 0.8) (layer "B.Cu") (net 6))
 (segment (start 170.7 86.75) (end 169.04 85.09) (width 0.8) (layer "B.Cu") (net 6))
 (segment (start 169.04 85.09) (end 154.915 85.09) (width 0.8) (layer "B.Cu") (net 6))
 (segment (start 141.3 90.67) (end 141.29 90.68) (width 0.4) (layer "F.Cu") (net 1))
 (segment (start 140.135 85.755) (end 144.72 85.755) (width 0.4) (layer "F.Cu") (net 1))
 (segment (start 145.385 85.09) (end 144.72 85.755) (width 0.4) (layer "F.Cu") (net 1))
 (segment (start 139.09 86.8) (end 140.135 85.755) (width 0.4) (layer "F.Cu") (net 1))
 (segment (start 139.09 90.04) (end 139.09 86.8) (width 0.4) (layer "F.Cu") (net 1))
 (segment (start 139.73 90.68) (end 139.09 90.04) (width 0.4) (layer "F.Cu") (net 1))
 (segment (start 141.29 90.68) (end 139.73 90.68) (width 0.4) (layer "F.Cu") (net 1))
 (segment (start 147.295 85.09) (end 145.385 85.09) (width 0.4) (layer "F.Cu") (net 1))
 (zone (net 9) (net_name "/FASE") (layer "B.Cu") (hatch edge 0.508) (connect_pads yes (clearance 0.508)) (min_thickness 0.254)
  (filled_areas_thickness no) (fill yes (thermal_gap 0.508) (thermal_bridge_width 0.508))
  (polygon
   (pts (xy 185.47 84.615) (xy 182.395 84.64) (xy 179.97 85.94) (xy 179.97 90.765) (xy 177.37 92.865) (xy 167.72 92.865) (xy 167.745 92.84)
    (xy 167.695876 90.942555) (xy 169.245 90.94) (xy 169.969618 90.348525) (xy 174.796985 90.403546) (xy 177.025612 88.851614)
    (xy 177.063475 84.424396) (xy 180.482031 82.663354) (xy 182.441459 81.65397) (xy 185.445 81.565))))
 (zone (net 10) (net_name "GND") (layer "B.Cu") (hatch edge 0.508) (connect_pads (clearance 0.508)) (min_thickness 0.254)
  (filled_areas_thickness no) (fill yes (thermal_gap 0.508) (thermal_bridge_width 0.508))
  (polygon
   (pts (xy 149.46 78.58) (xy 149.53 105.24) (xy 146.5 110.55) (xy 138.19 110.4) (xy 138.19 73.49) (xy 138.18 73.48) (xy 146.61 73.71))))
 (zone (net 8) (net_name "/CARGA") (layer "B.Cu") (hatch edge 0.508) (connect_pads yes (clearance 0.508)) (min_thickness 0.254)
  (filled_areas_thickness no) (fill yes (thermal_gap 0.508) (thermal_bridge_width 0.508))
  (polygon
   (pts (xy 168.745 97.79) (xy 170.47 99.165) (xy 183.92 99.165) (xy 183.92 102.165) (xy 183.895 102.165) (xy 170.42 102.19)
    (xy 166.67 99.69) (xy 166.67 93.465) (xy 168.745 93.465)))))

